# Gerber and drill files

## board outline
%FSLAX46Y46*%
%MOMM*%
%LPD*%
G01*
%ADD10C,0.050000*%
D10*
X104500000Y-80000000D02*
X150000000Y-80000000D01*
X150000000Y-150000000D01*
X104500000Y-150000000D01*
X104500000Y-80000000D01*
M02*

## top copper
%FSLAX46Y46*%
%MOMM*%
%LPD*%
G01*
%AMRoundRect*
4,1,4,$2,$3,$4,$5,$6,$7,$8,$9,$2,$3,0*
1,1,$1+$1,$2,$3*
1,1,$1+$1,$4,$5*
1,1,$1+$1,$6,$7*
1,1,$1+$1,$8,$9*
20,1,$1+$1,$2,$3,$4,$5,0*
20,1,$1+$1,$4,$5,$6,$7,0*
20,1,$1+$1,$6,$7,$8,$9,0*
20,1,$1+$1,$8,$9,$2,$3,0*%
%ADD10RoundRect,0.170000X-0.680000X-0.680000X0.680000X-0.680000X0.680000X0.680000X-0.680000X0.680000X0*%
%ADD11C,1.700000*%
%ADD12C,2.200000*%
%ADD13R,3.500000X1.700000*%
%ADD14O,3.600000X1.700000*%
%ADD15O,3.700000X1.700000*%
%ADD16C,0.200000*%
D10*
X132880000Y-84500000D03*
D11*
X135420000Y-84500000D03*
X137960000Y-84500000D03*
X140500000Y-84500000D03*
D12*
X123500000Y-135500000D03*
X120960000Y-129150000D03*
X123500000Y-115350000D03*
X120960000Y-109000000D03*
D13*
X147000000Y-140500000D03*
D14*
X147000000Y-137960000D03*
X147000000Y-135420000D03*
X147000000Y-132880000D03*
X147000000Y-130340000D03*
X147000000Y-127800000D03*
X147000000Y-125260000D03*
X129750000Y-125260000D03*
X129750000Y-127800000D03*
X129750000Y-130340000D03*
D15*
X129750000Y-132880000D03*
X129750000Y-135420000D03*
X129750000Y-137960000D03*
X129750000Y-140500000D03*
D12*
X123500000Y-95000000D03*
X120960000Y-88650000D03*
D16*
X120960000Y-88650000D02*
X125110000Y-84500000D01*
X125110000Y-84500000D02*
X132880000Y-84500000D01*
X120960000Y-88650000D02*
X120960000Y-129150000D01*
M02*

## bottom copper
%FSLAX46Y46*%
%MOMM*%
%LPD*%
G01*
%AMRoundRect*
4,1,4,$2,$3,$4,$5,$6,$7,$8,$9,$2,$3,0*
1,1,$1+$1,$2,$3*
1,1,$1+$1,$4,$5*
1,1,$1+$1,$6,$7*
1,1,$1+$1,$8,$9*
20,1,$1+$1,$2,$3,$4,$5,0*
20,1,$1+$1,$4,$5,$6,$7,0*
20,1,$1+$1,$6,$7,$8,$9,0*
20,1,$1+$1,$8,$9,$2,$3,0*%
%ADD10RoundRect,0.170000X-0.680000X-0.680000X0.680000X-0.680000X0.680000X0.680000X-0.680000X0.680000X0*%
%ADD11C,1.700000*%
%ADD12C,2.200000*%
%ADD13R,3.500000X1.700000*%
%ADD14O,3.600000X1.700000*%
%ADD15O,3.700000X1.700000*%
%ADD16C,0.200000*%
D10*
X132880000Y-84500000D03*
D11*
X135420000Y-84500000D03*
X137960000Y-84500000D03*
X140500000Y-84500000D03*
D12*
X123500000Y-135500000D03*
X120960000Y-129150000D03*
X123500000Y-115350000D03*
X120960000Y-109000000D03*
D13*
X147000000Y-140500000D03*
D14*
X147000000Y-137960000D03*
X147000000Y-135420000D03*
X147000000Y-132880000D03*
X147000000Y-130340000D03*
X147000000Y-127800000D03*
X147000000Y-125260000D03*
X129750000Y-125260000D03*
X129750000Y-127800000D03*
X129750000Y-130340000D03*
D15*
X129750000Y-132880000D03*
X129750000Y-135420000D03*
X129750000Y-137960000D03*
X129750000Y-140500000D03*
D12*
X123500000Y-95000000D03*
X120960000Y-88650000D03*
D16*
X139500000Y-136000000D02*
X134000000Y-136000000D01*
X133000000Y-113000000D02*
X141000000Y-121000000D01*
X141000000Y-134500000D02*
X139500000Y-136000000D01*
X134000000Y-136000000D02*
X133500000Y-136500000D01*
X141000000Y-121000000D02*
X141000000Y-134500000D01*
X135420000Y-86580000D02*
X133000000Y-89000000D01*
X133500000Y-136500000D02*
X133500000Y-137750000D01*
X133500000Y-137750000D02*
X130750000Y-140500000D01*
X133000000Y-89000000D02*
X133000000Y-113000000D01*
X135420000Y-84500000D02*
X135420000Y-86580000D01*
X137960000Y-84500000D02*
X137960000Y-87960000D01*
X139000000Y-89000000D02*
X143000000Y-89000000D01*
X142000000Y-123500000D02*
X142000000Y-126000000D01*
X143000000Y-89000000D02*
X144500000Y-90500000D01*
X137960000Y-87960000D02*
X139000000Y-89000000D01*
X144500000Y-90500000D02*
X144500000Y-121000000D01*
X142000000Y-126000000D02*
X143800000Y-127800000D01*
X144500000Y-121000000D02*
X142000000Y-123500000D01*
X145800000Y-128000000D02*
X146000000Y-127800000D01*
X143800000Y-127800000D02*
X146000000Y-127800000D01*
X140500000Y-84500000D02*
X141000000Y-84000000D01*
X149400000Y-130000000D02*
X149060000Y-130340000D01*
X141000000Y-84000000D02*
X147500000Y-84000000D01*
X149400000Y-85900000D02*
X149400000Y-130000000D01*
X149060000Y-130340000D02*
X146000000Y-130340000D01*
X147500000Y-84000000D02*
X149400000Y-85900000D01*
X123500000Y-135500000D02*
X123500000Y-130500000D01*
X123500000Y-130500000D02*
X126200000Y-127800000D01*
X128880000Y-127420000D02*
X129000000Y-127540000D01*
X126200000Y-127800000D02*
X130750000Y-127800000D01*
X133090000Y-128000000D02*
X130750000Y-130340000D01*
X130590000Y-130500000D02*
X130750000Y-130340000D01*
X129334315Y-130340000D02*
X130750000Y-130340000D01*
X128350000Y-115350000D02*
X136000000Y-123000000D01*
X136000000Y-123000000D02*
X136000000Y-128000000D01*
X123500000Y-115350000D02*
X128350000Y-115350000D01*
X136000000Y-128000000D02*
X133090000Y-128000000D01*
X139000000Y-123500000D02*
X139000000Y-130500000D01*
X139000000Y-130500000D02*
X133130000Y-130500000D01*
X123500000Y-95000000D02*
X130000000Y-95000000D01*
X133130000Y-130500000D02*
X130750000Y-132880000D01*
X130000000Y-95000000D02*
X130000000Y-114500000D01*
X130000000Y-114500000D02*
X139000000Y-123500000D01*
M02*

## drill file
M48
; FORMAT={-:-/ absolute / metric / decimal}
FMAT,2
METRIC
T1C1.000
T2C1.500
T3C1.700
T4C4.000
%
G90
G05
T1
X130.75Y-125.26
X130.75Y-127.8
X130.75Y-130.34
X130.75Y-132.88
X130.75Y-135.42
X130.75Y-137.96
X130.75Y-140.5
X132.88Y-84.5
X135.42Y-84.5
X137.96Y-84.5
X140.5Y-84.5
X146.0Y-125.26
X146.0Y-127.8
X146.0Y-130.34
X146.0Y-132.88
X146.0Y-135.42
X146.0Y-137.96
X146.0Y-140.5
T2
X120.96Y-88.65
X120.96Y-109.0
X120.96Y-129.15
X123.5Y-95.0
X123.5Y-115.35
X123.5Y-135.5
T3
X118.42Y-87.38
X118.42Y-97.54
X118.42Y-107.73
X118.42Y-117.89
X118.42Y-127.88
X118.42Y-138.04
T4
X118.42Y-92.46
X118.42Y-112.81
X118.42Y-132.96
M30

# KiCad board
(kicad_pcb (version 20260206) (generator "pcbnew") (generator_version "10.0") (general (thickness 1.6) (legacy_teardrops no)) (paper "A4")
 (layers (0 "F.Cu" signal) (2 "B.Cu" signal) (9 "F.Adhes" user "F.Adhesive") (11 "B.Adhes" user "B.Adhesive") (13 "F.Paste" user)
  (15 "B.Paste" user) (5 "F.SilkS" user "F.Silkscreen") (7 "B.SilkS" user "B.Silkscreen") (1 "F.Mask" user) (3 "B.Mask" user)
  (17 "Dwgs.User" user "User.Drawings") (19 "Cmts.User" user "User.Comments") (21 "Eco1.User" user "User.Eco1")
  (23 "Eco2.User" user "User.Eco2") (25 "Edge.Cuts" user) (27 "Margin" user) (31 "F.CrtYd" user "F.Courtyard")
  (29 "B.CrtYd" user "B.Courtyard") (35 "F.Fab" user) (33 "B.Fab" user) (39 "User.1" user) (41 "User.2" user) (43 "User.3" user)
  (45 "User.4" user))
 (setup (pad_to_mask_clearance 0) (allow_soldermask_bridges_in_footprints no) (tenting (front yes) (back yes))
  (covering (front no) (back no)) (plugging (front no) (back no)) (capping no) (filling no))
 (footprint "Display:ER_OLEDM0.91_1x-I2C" (layer "F.Cu") (at 132.88 84.5)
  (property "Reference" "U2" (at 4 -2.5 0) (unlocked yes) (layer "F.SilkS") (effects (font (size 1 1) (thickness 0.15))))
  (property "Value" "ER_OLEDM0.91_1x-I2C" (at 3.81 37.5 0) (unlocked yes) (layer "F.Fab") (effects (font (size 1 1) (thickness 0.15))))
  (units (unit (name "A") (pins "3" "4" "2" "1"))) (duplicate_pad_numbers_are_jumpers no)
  (pad "1" thru_hole roundrect (at 0 0) (size 1.7 1.7) (drill 1) (layers "*.Cu" "*.Mask") (remove_unused_layers no) (roundrect_rratio 0.1)
   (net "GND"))
  (pad "2" thru_hole circle (at 2.54 0) (size 1.7 1.7) (drill 1) (layers "*.Cu" "*.Mask") (remove_unused_layers no) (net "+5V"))
  (pad "3" thru_hole circle (at 5.08 0) (size 1.7 1.7) (drill 1) (layers "*.Cu" "*.Mask") (remove_unused_layers no)
   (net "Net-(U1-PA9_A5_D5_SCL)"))
  (pad "4" thru_hole circle (at 7.62 0) (size 1.7 1.7) (drill 1) (layers "*.Cu" "*.Mask") (remove_unused_layers no)
   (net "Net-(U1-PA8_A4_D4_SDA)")))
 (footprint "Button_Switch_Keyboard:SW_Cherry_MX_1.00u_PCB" (layer "F.Cu") (at 123.5 135.5 -90)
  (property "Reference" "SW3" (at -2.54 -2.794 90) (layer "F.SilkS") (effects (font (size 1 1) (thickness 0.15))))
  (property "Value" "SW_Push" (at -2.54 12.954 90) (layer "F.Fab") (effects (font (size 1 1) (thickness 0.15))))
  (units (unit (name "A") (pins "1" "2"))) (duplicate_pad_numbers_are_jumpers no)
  (pad "" np_thru_hole circle (at -7.62 5.08 270) (size 1.7 1.7) (drill 1.7) (layers "*.Cu" "*.Mask"))
  (pad "" np_thru_hole circle (at -2.54 5.08 270) (size 4 4) (drill 4) (layers "*.Cu" "*.Mask"))
  (pad "" np_thru_hole circle (at 2.54 5.08 270) (size 1.7 1.7) (drill 1.7) (layers "*.Cu" "*.Mask"))
  (pad "1" thru_hole circle (at 0 0 270) (size 2.2 2.2) (drill 1.5) (layers "*.Cu" "*.Mask") (remove_unused_layers no)
   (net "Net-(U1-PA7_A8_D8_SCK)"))
  (pad "2" thru_hole circle (at -6.35 2.54 270) (size 2.2 2.2) (drill 1.5) (layers "*.Cu" "*.Mask") (remove_unused_layers no) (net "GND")))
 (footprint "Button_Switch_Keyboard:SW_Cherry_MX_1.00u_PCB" (layer "F.Cu") (at 123.5 115.35 -90)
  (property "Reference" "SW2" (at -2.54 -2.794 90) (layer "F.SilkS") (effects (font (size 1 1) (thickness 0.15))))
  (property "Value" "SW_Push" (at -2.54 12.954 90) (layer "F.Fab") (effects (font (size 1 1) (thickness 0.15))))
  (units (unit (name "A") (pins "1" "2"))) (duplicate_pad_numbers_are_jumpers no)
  (pad "" np_thru_hole circle (at -7.62 5.08 270) (size 1.7 1.7) (drill 1.7) (layers "*.Cu" "*.Mask"))
  (pad "" np_thru_hole circle (at -2.54 5.08 270) (size 4 4) (drill 4) (layers "*.Cu" "*.Mask"))
  (pad "" np_thru_hole circle (at 2.54 5.08 270) (size 1.7 1.7) (drill 1.7) (layers "*.Cu" "*.Mask"))
  (pad "1" thru_hole circle (at 0 0 270) (size 2.2 2.2) (drill 1.5) (layers "*.Cu" "*.Mask") (remove_unused_layers no)
   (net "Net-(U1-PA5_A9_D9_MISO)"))
  (pad "2" thru_hole circle (at -6.35 2.54 270) (size 2.2 2.2) (drill 1.5) (layers "*.Cu" "*.Mask") (remove_unused_layers no) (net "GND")))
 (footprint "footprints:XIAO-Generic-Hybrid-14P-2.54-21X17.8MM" (layer "F.Cu") (at 138.375 132.88 180)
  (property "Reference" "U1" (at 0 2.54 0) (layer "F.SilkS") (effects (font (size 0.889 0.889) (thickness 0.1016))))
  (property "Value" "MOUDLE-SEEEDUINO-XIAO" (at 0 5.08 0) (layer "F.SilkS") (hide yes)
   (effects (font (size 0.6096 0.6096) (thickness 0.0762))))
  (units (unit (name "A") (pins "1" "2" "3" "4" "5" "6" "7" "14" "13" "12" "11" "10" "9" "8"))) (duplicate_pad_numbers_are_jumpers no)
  (pad "1" thru_hole rect (at -7.625 -7.62 180) (size 3.5 1.7) (drill 1 (offset -1 0)) (layers "*.Cu" "*.Mask") (remove_unused_layers no)
   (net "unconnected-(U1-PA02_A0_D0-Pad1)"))
  (pad "2" thru_hole oval (at -7.625 -5.08 180) (size 3.6 1.7) (drill 1 (offset -1 0)) (layers "*.Cu" "*.Mask") (remove_unused_layers no)
   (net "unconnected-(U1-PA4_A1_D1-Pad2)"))
  (pad "3" thru_hole oval (at -7.625 -2.54 180) (size 3.6 1.7) (drill 1 (offset -1 0)) (layers "*.Cu" "*.Mask") (remove_unused_layers no)
   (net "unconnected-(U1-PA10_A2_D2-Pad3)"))
  (pad "4" thru_hole oval (at -7.625 0 180) (size 3.6 1.7) (drill 1 (offset -1 0)) (layers "*.Cu" "*.Mask") (remove_unused_layers no)
   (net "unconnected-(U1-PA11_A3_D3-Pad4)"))
  (pad "5" thru_hole oval (at -7.625 2.54 180) (size 3.6 1.7) (drill 1 (offset -1 0)) (layers "*.Cu" "*.Mask") (remove_unused_layers no)
   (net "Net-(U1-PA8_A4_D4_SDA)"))
  (pad "6" thru_hole oval (at -7.625 5.08) (size 3.6 1.7) (drill 1 (offset 1 0)) (layers "*.Cu" "*.Mask") (remove_unused_layers no)
   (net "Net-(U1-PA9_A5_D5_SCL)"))
  (pad "7" thru_hole oval (at -7.625 7.62 180) (size 3.6 1.7) (drill 1 (offset -1 0)) (layers "*.Cu" "*.Mask") (remove_unused_layers no)
   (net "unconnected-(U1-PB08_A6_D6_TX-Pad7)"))
  (pad "8" thru_hole oval (at 7.625 7.62 180) (size 3.6 1.7) (drill 1 (offset 1 0)) (layers "*.Cu" "*.Mask") (remove_unused_layers no)
   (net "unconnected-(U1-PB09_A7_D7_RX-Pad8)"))
  (pad "9" thru_hole oval (at 7.625 5.08 180) (size 3.6 1.7) (drill 1 (offset 1 0)) (layers "*.Cu" "*.Mask") (remove_unused_layers no)
   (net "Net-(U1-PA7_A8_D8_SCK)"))
  (pad "10" thru_hole oval (at 7.625 2.54 180) (size 3.6 1.7) (drill 1 (offset 1 0)) (layers "*.Cu" "*.Mask") (remove_unused_layers no)
   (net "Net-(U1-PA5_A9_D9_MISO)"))
  (pad "11" thru_hole oval (at 7.625 0 180) (size 3.7 1.7) (drill 1 (offset 1 0)) (layers "*.Cu" "*.Mask") (remove_unused_layers no)
   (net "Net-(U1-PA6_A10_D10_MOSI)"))
  (pad "12" thru_hole oval (at 7.625 -2.54 180) (size 3.7 1.7) (drill 1 (offset 1 0)) (layers "*.Cu" "*.Mask") (remove_unused_layers no)
   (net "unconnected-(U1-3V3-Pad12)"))
  (pad "13" thru_hole oval (at 7.625 -5.08 180) (size 3.7 1.7) (drill 1 (offset 1 0)) (layers "*.Cu" "*.Mask") (remove_unused_layers no)
   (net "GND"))
  (pad "14" thru_hole oval (at 7.625 -7.62 180) (size 3.7 1.7) (drill 1 (offset 1 0)) (layers "*.Cu" "*.Mask") (remove_unused_layers no)
   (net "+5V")))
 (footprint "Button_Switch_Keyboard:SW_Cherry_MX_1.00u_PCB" (layer "F.Cu") (at 123.5 95 -90)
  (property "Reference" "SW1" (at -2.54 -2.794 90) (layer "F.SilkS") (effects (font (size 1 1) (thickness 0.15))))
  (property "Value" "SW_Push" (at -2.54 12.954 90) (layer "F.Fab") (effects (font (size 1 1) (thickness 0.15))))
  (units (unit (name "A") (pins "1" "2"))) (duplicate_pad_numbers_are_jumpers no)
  (pad "" np_thru_hole circle (at -7.62 5.08 270) (size 1.7 1.7) (drill 1.7) (layers "*.Cu" "*.Mask"))
  (pad "" np_thru_hole circle (at -2.54 5.08 270) (size 4 4) (drill 4) (layers "*.Cu" "*.Mask"))
  (pad "" np_thru_hole circle (at 2.54 5.08 270) (size 1.7 1.7) (drill 1.7) (layers "*.Cu" "*.Mask"))
  (pad "1" thru_hole circle (at 0 0 270) (size 2.2 2.2) (drill 1.5) (layers "*.Cu" "*.Mask") (remove_unused_layers no)
   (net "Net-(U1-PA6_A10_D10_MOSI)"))
  (pad "2" thru_hole circle (at -6.35 2.54 270) (size 2.2 2.2) (drill 1.5) (layers "*.Cu" "*.Mask") (remove_unused_layers no) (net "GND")))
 (gr_rect (start 104.5 80) (end 150 150) (stroke (width 0.05) (type default)) (fill no) (layer "Edge.Cuts"))
 (segment (start 120.96 88.65) (end 125.11 84.5) (width 0.2) (layer "F.Cu") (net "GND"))
 (segment (start 125.11 84.5) (end 132.88 84.5) (width 0.2) (layer "F.Cu") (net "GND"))
 (segment (start 120.96 88.65) (end 120.96 129.15) (width 0.2) (layer "F.Cu") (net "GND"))
 (segment (start 139.5 136) (end 134 136) (width 0.2) (layer "B.Cu") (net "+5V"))
 (segment (start 133 113) (end 141 121) (width 0.2) (layer "B.Cu") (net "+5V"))
 (segment (start 141 134.5) (end 139.5 136) (width 0.2) (layer "B.Cu") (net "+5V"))
 (segment (start 134 136) (end 133.5 136.5) (width 0.2) (layer "B.Cu") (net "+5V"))
 (segment (start 141 121) (end 141 134.5) (width 0.2) (layer "B.Cu") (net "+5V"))
 (segment (start 135.42 86.58) (end 133 89) (width 0.2) (layer "B.Cu") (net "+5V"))
 (segment (start 133.5 136.5) (end 133.5 137.75) (width 0.2) (layer "B.Cu") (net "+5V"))
 (segment (start 133.5 137.75) (end 130.75 140.5) (width 0.2) (layer "B.Cu") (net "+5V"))
 (segment (start 133 89) (end 133 113) (width 0.2) (layer "B.Cu") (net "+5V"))
 (segment (start 135.42 84.5) (end 135.42 86.58) (width 0.2) (layer "B.Cu") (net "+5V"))
 (segment (start 137.96 84.5) (end 137.96 87.96) (width 0.2) (layer "B.Cu") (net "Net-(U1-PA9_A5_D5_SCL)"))
 (segment (start 139 89) (end 143 89) (width 0.2) (layer "B.Cu") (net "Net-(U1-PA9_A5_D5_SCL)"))
 (segment (start 142 123.5) (end 142 126) (width 0.2) (layer "B.Cu") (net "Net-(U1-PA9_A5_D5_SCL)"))
 (segment (start 143 89) (end 144.5 90.5) (width 0.2) (layer "B.Cu") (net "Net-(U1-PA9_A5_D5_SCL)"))
 (segment (start 137.96 87.96) (end 139 89) (width 0.2) (layer "B.Cu") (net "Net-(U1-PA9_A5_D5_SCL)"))
 (segment (start 144.5 90.5) (end 144.5 121) (width 0.2) (layer "B.Cu") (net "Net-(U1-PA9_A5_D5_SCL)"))
 (segment (start 142 126) (end 143.8 127.8) (width 0.2) (layer "B.Cu") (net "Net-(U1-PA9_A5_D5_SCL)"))
 (segment (start 144.5 121) (end 142 123.5) (width 0.2) (layer "B.Cu") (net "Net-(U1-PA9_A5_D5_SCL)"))
 (segment (start 145.8 128) (end 146 127.8) (width 0.2) (layer "B.Cu") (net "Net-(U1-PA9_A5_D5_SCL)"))
 (segment (start 143.8 127.8) (end 146 127.8) (width 0.2) (layer "B.Cu") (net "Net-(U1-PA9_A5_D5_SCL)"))
 (segment (start 140.5 84.5) (end 141 84) (width 0.2) (layer "B.Cu") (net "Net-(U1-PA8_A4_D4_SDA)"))
 (segment (start 149.4 130) (end 149.06 130.34) (width 0.2) (layer "B.Cu") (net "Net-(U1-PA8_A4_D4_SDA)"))
 (segment (start 141 84) (end 147.5 84) (width 0.2) (layer "B.Cu") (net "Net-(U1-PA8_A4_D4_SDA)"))
 (segment (start 149.4 85.9) (end 149.4 130) (width 0.2) (layer "B.Cu") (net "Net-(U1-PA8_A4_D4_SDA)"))
 (segment (start 149.06 130.34) (end 146 130.34) (width 0.2) (layer "B.Cu") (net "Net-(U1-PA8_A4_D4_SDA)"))
 (segment (start 147.5 84) (end 149.4 85.9) (width 0.2) (layer "B.Cu") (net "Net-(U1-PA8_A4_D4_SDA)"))
 (segment (start 123.5 135.5) (end 123.5 130.5) (width 0.2) (layer "B.Cu") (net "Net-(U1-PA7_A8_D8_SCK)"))
 (segment (start 123.5 130.5) (end 126.2 127.8) (width 0.2) (layer "B.Cu") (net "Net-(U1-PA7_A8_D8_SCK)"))
 (segment (start 128.88 127.42) (end 129 127.54) (width 0.2) (layer "B.Cu") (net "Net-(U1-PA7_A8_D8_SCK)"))
 (segment (start 126.2 127.8) (end 130.75 127.8) (width 0.2) (layer "B.Cu") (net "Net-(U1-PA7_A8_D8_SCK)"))
 (segment (start 133.09 128) (end 130.75 130.34) (width 0.2) (layer "B.Cu") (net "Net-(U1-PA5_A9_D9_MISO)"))
 (segment (start 130.59 130.5) (end 130.75 130.34) (width 0.2) (layer "B.Cu") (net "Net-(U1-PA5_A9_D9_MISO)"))
 (segment (start 129.334315 130.34) (end 130.75 130.34) (width 0.2) (layer "B.Cu") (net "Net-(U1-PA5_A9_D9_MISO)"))
 (segment (start 128.35 115.35) (end 136 123) (width 0.2) (layer "B.Cu") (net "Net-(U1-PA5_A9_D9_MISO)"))
 (segment (start 136 123) (end 136 128) (width 0.2) (layer "B.Cu") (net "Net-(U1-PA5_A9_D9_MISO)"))
 (segment (start 123.5 115.35) (end 128.35 115.35) (width 0.2) (layer "B.Cu") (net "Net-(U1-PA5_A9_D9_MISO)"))
 (segment (start 136 128) (end 133.09 128) (width 0.2) (layer "B.Cu") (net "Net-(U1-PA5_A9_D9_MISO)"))
 (segment (start 139 123.5) (end 139 130.5) (width 0.2) (layer "B.Cu") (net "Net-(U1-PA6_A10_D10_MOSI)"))
 (segment (start 139 130.5) (end 133.13 130.5) (width 0.2) (layer "B.Cu") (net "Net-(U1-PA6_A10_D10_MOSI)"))
 (segment (start 123.5 95) (end 130 95) (width 0.2) (layer "B.Cu") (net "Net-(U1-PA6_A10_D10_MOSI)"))
 (segment (start 133.13 130.5) (end 130.75 132.88) (width 0.2) (layer "B.Cu") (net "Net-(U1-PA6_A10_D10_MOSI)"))
 (segment (start 130 95) (end 130 114.5) (width 0.2) (layer "B.Cu") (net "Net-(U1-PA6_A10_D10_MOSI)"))
 (segment (start 130 114.5) (end 139 123.5) (width 0.2) (layer "B.Cu") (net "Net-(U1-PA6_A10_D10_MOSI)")))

